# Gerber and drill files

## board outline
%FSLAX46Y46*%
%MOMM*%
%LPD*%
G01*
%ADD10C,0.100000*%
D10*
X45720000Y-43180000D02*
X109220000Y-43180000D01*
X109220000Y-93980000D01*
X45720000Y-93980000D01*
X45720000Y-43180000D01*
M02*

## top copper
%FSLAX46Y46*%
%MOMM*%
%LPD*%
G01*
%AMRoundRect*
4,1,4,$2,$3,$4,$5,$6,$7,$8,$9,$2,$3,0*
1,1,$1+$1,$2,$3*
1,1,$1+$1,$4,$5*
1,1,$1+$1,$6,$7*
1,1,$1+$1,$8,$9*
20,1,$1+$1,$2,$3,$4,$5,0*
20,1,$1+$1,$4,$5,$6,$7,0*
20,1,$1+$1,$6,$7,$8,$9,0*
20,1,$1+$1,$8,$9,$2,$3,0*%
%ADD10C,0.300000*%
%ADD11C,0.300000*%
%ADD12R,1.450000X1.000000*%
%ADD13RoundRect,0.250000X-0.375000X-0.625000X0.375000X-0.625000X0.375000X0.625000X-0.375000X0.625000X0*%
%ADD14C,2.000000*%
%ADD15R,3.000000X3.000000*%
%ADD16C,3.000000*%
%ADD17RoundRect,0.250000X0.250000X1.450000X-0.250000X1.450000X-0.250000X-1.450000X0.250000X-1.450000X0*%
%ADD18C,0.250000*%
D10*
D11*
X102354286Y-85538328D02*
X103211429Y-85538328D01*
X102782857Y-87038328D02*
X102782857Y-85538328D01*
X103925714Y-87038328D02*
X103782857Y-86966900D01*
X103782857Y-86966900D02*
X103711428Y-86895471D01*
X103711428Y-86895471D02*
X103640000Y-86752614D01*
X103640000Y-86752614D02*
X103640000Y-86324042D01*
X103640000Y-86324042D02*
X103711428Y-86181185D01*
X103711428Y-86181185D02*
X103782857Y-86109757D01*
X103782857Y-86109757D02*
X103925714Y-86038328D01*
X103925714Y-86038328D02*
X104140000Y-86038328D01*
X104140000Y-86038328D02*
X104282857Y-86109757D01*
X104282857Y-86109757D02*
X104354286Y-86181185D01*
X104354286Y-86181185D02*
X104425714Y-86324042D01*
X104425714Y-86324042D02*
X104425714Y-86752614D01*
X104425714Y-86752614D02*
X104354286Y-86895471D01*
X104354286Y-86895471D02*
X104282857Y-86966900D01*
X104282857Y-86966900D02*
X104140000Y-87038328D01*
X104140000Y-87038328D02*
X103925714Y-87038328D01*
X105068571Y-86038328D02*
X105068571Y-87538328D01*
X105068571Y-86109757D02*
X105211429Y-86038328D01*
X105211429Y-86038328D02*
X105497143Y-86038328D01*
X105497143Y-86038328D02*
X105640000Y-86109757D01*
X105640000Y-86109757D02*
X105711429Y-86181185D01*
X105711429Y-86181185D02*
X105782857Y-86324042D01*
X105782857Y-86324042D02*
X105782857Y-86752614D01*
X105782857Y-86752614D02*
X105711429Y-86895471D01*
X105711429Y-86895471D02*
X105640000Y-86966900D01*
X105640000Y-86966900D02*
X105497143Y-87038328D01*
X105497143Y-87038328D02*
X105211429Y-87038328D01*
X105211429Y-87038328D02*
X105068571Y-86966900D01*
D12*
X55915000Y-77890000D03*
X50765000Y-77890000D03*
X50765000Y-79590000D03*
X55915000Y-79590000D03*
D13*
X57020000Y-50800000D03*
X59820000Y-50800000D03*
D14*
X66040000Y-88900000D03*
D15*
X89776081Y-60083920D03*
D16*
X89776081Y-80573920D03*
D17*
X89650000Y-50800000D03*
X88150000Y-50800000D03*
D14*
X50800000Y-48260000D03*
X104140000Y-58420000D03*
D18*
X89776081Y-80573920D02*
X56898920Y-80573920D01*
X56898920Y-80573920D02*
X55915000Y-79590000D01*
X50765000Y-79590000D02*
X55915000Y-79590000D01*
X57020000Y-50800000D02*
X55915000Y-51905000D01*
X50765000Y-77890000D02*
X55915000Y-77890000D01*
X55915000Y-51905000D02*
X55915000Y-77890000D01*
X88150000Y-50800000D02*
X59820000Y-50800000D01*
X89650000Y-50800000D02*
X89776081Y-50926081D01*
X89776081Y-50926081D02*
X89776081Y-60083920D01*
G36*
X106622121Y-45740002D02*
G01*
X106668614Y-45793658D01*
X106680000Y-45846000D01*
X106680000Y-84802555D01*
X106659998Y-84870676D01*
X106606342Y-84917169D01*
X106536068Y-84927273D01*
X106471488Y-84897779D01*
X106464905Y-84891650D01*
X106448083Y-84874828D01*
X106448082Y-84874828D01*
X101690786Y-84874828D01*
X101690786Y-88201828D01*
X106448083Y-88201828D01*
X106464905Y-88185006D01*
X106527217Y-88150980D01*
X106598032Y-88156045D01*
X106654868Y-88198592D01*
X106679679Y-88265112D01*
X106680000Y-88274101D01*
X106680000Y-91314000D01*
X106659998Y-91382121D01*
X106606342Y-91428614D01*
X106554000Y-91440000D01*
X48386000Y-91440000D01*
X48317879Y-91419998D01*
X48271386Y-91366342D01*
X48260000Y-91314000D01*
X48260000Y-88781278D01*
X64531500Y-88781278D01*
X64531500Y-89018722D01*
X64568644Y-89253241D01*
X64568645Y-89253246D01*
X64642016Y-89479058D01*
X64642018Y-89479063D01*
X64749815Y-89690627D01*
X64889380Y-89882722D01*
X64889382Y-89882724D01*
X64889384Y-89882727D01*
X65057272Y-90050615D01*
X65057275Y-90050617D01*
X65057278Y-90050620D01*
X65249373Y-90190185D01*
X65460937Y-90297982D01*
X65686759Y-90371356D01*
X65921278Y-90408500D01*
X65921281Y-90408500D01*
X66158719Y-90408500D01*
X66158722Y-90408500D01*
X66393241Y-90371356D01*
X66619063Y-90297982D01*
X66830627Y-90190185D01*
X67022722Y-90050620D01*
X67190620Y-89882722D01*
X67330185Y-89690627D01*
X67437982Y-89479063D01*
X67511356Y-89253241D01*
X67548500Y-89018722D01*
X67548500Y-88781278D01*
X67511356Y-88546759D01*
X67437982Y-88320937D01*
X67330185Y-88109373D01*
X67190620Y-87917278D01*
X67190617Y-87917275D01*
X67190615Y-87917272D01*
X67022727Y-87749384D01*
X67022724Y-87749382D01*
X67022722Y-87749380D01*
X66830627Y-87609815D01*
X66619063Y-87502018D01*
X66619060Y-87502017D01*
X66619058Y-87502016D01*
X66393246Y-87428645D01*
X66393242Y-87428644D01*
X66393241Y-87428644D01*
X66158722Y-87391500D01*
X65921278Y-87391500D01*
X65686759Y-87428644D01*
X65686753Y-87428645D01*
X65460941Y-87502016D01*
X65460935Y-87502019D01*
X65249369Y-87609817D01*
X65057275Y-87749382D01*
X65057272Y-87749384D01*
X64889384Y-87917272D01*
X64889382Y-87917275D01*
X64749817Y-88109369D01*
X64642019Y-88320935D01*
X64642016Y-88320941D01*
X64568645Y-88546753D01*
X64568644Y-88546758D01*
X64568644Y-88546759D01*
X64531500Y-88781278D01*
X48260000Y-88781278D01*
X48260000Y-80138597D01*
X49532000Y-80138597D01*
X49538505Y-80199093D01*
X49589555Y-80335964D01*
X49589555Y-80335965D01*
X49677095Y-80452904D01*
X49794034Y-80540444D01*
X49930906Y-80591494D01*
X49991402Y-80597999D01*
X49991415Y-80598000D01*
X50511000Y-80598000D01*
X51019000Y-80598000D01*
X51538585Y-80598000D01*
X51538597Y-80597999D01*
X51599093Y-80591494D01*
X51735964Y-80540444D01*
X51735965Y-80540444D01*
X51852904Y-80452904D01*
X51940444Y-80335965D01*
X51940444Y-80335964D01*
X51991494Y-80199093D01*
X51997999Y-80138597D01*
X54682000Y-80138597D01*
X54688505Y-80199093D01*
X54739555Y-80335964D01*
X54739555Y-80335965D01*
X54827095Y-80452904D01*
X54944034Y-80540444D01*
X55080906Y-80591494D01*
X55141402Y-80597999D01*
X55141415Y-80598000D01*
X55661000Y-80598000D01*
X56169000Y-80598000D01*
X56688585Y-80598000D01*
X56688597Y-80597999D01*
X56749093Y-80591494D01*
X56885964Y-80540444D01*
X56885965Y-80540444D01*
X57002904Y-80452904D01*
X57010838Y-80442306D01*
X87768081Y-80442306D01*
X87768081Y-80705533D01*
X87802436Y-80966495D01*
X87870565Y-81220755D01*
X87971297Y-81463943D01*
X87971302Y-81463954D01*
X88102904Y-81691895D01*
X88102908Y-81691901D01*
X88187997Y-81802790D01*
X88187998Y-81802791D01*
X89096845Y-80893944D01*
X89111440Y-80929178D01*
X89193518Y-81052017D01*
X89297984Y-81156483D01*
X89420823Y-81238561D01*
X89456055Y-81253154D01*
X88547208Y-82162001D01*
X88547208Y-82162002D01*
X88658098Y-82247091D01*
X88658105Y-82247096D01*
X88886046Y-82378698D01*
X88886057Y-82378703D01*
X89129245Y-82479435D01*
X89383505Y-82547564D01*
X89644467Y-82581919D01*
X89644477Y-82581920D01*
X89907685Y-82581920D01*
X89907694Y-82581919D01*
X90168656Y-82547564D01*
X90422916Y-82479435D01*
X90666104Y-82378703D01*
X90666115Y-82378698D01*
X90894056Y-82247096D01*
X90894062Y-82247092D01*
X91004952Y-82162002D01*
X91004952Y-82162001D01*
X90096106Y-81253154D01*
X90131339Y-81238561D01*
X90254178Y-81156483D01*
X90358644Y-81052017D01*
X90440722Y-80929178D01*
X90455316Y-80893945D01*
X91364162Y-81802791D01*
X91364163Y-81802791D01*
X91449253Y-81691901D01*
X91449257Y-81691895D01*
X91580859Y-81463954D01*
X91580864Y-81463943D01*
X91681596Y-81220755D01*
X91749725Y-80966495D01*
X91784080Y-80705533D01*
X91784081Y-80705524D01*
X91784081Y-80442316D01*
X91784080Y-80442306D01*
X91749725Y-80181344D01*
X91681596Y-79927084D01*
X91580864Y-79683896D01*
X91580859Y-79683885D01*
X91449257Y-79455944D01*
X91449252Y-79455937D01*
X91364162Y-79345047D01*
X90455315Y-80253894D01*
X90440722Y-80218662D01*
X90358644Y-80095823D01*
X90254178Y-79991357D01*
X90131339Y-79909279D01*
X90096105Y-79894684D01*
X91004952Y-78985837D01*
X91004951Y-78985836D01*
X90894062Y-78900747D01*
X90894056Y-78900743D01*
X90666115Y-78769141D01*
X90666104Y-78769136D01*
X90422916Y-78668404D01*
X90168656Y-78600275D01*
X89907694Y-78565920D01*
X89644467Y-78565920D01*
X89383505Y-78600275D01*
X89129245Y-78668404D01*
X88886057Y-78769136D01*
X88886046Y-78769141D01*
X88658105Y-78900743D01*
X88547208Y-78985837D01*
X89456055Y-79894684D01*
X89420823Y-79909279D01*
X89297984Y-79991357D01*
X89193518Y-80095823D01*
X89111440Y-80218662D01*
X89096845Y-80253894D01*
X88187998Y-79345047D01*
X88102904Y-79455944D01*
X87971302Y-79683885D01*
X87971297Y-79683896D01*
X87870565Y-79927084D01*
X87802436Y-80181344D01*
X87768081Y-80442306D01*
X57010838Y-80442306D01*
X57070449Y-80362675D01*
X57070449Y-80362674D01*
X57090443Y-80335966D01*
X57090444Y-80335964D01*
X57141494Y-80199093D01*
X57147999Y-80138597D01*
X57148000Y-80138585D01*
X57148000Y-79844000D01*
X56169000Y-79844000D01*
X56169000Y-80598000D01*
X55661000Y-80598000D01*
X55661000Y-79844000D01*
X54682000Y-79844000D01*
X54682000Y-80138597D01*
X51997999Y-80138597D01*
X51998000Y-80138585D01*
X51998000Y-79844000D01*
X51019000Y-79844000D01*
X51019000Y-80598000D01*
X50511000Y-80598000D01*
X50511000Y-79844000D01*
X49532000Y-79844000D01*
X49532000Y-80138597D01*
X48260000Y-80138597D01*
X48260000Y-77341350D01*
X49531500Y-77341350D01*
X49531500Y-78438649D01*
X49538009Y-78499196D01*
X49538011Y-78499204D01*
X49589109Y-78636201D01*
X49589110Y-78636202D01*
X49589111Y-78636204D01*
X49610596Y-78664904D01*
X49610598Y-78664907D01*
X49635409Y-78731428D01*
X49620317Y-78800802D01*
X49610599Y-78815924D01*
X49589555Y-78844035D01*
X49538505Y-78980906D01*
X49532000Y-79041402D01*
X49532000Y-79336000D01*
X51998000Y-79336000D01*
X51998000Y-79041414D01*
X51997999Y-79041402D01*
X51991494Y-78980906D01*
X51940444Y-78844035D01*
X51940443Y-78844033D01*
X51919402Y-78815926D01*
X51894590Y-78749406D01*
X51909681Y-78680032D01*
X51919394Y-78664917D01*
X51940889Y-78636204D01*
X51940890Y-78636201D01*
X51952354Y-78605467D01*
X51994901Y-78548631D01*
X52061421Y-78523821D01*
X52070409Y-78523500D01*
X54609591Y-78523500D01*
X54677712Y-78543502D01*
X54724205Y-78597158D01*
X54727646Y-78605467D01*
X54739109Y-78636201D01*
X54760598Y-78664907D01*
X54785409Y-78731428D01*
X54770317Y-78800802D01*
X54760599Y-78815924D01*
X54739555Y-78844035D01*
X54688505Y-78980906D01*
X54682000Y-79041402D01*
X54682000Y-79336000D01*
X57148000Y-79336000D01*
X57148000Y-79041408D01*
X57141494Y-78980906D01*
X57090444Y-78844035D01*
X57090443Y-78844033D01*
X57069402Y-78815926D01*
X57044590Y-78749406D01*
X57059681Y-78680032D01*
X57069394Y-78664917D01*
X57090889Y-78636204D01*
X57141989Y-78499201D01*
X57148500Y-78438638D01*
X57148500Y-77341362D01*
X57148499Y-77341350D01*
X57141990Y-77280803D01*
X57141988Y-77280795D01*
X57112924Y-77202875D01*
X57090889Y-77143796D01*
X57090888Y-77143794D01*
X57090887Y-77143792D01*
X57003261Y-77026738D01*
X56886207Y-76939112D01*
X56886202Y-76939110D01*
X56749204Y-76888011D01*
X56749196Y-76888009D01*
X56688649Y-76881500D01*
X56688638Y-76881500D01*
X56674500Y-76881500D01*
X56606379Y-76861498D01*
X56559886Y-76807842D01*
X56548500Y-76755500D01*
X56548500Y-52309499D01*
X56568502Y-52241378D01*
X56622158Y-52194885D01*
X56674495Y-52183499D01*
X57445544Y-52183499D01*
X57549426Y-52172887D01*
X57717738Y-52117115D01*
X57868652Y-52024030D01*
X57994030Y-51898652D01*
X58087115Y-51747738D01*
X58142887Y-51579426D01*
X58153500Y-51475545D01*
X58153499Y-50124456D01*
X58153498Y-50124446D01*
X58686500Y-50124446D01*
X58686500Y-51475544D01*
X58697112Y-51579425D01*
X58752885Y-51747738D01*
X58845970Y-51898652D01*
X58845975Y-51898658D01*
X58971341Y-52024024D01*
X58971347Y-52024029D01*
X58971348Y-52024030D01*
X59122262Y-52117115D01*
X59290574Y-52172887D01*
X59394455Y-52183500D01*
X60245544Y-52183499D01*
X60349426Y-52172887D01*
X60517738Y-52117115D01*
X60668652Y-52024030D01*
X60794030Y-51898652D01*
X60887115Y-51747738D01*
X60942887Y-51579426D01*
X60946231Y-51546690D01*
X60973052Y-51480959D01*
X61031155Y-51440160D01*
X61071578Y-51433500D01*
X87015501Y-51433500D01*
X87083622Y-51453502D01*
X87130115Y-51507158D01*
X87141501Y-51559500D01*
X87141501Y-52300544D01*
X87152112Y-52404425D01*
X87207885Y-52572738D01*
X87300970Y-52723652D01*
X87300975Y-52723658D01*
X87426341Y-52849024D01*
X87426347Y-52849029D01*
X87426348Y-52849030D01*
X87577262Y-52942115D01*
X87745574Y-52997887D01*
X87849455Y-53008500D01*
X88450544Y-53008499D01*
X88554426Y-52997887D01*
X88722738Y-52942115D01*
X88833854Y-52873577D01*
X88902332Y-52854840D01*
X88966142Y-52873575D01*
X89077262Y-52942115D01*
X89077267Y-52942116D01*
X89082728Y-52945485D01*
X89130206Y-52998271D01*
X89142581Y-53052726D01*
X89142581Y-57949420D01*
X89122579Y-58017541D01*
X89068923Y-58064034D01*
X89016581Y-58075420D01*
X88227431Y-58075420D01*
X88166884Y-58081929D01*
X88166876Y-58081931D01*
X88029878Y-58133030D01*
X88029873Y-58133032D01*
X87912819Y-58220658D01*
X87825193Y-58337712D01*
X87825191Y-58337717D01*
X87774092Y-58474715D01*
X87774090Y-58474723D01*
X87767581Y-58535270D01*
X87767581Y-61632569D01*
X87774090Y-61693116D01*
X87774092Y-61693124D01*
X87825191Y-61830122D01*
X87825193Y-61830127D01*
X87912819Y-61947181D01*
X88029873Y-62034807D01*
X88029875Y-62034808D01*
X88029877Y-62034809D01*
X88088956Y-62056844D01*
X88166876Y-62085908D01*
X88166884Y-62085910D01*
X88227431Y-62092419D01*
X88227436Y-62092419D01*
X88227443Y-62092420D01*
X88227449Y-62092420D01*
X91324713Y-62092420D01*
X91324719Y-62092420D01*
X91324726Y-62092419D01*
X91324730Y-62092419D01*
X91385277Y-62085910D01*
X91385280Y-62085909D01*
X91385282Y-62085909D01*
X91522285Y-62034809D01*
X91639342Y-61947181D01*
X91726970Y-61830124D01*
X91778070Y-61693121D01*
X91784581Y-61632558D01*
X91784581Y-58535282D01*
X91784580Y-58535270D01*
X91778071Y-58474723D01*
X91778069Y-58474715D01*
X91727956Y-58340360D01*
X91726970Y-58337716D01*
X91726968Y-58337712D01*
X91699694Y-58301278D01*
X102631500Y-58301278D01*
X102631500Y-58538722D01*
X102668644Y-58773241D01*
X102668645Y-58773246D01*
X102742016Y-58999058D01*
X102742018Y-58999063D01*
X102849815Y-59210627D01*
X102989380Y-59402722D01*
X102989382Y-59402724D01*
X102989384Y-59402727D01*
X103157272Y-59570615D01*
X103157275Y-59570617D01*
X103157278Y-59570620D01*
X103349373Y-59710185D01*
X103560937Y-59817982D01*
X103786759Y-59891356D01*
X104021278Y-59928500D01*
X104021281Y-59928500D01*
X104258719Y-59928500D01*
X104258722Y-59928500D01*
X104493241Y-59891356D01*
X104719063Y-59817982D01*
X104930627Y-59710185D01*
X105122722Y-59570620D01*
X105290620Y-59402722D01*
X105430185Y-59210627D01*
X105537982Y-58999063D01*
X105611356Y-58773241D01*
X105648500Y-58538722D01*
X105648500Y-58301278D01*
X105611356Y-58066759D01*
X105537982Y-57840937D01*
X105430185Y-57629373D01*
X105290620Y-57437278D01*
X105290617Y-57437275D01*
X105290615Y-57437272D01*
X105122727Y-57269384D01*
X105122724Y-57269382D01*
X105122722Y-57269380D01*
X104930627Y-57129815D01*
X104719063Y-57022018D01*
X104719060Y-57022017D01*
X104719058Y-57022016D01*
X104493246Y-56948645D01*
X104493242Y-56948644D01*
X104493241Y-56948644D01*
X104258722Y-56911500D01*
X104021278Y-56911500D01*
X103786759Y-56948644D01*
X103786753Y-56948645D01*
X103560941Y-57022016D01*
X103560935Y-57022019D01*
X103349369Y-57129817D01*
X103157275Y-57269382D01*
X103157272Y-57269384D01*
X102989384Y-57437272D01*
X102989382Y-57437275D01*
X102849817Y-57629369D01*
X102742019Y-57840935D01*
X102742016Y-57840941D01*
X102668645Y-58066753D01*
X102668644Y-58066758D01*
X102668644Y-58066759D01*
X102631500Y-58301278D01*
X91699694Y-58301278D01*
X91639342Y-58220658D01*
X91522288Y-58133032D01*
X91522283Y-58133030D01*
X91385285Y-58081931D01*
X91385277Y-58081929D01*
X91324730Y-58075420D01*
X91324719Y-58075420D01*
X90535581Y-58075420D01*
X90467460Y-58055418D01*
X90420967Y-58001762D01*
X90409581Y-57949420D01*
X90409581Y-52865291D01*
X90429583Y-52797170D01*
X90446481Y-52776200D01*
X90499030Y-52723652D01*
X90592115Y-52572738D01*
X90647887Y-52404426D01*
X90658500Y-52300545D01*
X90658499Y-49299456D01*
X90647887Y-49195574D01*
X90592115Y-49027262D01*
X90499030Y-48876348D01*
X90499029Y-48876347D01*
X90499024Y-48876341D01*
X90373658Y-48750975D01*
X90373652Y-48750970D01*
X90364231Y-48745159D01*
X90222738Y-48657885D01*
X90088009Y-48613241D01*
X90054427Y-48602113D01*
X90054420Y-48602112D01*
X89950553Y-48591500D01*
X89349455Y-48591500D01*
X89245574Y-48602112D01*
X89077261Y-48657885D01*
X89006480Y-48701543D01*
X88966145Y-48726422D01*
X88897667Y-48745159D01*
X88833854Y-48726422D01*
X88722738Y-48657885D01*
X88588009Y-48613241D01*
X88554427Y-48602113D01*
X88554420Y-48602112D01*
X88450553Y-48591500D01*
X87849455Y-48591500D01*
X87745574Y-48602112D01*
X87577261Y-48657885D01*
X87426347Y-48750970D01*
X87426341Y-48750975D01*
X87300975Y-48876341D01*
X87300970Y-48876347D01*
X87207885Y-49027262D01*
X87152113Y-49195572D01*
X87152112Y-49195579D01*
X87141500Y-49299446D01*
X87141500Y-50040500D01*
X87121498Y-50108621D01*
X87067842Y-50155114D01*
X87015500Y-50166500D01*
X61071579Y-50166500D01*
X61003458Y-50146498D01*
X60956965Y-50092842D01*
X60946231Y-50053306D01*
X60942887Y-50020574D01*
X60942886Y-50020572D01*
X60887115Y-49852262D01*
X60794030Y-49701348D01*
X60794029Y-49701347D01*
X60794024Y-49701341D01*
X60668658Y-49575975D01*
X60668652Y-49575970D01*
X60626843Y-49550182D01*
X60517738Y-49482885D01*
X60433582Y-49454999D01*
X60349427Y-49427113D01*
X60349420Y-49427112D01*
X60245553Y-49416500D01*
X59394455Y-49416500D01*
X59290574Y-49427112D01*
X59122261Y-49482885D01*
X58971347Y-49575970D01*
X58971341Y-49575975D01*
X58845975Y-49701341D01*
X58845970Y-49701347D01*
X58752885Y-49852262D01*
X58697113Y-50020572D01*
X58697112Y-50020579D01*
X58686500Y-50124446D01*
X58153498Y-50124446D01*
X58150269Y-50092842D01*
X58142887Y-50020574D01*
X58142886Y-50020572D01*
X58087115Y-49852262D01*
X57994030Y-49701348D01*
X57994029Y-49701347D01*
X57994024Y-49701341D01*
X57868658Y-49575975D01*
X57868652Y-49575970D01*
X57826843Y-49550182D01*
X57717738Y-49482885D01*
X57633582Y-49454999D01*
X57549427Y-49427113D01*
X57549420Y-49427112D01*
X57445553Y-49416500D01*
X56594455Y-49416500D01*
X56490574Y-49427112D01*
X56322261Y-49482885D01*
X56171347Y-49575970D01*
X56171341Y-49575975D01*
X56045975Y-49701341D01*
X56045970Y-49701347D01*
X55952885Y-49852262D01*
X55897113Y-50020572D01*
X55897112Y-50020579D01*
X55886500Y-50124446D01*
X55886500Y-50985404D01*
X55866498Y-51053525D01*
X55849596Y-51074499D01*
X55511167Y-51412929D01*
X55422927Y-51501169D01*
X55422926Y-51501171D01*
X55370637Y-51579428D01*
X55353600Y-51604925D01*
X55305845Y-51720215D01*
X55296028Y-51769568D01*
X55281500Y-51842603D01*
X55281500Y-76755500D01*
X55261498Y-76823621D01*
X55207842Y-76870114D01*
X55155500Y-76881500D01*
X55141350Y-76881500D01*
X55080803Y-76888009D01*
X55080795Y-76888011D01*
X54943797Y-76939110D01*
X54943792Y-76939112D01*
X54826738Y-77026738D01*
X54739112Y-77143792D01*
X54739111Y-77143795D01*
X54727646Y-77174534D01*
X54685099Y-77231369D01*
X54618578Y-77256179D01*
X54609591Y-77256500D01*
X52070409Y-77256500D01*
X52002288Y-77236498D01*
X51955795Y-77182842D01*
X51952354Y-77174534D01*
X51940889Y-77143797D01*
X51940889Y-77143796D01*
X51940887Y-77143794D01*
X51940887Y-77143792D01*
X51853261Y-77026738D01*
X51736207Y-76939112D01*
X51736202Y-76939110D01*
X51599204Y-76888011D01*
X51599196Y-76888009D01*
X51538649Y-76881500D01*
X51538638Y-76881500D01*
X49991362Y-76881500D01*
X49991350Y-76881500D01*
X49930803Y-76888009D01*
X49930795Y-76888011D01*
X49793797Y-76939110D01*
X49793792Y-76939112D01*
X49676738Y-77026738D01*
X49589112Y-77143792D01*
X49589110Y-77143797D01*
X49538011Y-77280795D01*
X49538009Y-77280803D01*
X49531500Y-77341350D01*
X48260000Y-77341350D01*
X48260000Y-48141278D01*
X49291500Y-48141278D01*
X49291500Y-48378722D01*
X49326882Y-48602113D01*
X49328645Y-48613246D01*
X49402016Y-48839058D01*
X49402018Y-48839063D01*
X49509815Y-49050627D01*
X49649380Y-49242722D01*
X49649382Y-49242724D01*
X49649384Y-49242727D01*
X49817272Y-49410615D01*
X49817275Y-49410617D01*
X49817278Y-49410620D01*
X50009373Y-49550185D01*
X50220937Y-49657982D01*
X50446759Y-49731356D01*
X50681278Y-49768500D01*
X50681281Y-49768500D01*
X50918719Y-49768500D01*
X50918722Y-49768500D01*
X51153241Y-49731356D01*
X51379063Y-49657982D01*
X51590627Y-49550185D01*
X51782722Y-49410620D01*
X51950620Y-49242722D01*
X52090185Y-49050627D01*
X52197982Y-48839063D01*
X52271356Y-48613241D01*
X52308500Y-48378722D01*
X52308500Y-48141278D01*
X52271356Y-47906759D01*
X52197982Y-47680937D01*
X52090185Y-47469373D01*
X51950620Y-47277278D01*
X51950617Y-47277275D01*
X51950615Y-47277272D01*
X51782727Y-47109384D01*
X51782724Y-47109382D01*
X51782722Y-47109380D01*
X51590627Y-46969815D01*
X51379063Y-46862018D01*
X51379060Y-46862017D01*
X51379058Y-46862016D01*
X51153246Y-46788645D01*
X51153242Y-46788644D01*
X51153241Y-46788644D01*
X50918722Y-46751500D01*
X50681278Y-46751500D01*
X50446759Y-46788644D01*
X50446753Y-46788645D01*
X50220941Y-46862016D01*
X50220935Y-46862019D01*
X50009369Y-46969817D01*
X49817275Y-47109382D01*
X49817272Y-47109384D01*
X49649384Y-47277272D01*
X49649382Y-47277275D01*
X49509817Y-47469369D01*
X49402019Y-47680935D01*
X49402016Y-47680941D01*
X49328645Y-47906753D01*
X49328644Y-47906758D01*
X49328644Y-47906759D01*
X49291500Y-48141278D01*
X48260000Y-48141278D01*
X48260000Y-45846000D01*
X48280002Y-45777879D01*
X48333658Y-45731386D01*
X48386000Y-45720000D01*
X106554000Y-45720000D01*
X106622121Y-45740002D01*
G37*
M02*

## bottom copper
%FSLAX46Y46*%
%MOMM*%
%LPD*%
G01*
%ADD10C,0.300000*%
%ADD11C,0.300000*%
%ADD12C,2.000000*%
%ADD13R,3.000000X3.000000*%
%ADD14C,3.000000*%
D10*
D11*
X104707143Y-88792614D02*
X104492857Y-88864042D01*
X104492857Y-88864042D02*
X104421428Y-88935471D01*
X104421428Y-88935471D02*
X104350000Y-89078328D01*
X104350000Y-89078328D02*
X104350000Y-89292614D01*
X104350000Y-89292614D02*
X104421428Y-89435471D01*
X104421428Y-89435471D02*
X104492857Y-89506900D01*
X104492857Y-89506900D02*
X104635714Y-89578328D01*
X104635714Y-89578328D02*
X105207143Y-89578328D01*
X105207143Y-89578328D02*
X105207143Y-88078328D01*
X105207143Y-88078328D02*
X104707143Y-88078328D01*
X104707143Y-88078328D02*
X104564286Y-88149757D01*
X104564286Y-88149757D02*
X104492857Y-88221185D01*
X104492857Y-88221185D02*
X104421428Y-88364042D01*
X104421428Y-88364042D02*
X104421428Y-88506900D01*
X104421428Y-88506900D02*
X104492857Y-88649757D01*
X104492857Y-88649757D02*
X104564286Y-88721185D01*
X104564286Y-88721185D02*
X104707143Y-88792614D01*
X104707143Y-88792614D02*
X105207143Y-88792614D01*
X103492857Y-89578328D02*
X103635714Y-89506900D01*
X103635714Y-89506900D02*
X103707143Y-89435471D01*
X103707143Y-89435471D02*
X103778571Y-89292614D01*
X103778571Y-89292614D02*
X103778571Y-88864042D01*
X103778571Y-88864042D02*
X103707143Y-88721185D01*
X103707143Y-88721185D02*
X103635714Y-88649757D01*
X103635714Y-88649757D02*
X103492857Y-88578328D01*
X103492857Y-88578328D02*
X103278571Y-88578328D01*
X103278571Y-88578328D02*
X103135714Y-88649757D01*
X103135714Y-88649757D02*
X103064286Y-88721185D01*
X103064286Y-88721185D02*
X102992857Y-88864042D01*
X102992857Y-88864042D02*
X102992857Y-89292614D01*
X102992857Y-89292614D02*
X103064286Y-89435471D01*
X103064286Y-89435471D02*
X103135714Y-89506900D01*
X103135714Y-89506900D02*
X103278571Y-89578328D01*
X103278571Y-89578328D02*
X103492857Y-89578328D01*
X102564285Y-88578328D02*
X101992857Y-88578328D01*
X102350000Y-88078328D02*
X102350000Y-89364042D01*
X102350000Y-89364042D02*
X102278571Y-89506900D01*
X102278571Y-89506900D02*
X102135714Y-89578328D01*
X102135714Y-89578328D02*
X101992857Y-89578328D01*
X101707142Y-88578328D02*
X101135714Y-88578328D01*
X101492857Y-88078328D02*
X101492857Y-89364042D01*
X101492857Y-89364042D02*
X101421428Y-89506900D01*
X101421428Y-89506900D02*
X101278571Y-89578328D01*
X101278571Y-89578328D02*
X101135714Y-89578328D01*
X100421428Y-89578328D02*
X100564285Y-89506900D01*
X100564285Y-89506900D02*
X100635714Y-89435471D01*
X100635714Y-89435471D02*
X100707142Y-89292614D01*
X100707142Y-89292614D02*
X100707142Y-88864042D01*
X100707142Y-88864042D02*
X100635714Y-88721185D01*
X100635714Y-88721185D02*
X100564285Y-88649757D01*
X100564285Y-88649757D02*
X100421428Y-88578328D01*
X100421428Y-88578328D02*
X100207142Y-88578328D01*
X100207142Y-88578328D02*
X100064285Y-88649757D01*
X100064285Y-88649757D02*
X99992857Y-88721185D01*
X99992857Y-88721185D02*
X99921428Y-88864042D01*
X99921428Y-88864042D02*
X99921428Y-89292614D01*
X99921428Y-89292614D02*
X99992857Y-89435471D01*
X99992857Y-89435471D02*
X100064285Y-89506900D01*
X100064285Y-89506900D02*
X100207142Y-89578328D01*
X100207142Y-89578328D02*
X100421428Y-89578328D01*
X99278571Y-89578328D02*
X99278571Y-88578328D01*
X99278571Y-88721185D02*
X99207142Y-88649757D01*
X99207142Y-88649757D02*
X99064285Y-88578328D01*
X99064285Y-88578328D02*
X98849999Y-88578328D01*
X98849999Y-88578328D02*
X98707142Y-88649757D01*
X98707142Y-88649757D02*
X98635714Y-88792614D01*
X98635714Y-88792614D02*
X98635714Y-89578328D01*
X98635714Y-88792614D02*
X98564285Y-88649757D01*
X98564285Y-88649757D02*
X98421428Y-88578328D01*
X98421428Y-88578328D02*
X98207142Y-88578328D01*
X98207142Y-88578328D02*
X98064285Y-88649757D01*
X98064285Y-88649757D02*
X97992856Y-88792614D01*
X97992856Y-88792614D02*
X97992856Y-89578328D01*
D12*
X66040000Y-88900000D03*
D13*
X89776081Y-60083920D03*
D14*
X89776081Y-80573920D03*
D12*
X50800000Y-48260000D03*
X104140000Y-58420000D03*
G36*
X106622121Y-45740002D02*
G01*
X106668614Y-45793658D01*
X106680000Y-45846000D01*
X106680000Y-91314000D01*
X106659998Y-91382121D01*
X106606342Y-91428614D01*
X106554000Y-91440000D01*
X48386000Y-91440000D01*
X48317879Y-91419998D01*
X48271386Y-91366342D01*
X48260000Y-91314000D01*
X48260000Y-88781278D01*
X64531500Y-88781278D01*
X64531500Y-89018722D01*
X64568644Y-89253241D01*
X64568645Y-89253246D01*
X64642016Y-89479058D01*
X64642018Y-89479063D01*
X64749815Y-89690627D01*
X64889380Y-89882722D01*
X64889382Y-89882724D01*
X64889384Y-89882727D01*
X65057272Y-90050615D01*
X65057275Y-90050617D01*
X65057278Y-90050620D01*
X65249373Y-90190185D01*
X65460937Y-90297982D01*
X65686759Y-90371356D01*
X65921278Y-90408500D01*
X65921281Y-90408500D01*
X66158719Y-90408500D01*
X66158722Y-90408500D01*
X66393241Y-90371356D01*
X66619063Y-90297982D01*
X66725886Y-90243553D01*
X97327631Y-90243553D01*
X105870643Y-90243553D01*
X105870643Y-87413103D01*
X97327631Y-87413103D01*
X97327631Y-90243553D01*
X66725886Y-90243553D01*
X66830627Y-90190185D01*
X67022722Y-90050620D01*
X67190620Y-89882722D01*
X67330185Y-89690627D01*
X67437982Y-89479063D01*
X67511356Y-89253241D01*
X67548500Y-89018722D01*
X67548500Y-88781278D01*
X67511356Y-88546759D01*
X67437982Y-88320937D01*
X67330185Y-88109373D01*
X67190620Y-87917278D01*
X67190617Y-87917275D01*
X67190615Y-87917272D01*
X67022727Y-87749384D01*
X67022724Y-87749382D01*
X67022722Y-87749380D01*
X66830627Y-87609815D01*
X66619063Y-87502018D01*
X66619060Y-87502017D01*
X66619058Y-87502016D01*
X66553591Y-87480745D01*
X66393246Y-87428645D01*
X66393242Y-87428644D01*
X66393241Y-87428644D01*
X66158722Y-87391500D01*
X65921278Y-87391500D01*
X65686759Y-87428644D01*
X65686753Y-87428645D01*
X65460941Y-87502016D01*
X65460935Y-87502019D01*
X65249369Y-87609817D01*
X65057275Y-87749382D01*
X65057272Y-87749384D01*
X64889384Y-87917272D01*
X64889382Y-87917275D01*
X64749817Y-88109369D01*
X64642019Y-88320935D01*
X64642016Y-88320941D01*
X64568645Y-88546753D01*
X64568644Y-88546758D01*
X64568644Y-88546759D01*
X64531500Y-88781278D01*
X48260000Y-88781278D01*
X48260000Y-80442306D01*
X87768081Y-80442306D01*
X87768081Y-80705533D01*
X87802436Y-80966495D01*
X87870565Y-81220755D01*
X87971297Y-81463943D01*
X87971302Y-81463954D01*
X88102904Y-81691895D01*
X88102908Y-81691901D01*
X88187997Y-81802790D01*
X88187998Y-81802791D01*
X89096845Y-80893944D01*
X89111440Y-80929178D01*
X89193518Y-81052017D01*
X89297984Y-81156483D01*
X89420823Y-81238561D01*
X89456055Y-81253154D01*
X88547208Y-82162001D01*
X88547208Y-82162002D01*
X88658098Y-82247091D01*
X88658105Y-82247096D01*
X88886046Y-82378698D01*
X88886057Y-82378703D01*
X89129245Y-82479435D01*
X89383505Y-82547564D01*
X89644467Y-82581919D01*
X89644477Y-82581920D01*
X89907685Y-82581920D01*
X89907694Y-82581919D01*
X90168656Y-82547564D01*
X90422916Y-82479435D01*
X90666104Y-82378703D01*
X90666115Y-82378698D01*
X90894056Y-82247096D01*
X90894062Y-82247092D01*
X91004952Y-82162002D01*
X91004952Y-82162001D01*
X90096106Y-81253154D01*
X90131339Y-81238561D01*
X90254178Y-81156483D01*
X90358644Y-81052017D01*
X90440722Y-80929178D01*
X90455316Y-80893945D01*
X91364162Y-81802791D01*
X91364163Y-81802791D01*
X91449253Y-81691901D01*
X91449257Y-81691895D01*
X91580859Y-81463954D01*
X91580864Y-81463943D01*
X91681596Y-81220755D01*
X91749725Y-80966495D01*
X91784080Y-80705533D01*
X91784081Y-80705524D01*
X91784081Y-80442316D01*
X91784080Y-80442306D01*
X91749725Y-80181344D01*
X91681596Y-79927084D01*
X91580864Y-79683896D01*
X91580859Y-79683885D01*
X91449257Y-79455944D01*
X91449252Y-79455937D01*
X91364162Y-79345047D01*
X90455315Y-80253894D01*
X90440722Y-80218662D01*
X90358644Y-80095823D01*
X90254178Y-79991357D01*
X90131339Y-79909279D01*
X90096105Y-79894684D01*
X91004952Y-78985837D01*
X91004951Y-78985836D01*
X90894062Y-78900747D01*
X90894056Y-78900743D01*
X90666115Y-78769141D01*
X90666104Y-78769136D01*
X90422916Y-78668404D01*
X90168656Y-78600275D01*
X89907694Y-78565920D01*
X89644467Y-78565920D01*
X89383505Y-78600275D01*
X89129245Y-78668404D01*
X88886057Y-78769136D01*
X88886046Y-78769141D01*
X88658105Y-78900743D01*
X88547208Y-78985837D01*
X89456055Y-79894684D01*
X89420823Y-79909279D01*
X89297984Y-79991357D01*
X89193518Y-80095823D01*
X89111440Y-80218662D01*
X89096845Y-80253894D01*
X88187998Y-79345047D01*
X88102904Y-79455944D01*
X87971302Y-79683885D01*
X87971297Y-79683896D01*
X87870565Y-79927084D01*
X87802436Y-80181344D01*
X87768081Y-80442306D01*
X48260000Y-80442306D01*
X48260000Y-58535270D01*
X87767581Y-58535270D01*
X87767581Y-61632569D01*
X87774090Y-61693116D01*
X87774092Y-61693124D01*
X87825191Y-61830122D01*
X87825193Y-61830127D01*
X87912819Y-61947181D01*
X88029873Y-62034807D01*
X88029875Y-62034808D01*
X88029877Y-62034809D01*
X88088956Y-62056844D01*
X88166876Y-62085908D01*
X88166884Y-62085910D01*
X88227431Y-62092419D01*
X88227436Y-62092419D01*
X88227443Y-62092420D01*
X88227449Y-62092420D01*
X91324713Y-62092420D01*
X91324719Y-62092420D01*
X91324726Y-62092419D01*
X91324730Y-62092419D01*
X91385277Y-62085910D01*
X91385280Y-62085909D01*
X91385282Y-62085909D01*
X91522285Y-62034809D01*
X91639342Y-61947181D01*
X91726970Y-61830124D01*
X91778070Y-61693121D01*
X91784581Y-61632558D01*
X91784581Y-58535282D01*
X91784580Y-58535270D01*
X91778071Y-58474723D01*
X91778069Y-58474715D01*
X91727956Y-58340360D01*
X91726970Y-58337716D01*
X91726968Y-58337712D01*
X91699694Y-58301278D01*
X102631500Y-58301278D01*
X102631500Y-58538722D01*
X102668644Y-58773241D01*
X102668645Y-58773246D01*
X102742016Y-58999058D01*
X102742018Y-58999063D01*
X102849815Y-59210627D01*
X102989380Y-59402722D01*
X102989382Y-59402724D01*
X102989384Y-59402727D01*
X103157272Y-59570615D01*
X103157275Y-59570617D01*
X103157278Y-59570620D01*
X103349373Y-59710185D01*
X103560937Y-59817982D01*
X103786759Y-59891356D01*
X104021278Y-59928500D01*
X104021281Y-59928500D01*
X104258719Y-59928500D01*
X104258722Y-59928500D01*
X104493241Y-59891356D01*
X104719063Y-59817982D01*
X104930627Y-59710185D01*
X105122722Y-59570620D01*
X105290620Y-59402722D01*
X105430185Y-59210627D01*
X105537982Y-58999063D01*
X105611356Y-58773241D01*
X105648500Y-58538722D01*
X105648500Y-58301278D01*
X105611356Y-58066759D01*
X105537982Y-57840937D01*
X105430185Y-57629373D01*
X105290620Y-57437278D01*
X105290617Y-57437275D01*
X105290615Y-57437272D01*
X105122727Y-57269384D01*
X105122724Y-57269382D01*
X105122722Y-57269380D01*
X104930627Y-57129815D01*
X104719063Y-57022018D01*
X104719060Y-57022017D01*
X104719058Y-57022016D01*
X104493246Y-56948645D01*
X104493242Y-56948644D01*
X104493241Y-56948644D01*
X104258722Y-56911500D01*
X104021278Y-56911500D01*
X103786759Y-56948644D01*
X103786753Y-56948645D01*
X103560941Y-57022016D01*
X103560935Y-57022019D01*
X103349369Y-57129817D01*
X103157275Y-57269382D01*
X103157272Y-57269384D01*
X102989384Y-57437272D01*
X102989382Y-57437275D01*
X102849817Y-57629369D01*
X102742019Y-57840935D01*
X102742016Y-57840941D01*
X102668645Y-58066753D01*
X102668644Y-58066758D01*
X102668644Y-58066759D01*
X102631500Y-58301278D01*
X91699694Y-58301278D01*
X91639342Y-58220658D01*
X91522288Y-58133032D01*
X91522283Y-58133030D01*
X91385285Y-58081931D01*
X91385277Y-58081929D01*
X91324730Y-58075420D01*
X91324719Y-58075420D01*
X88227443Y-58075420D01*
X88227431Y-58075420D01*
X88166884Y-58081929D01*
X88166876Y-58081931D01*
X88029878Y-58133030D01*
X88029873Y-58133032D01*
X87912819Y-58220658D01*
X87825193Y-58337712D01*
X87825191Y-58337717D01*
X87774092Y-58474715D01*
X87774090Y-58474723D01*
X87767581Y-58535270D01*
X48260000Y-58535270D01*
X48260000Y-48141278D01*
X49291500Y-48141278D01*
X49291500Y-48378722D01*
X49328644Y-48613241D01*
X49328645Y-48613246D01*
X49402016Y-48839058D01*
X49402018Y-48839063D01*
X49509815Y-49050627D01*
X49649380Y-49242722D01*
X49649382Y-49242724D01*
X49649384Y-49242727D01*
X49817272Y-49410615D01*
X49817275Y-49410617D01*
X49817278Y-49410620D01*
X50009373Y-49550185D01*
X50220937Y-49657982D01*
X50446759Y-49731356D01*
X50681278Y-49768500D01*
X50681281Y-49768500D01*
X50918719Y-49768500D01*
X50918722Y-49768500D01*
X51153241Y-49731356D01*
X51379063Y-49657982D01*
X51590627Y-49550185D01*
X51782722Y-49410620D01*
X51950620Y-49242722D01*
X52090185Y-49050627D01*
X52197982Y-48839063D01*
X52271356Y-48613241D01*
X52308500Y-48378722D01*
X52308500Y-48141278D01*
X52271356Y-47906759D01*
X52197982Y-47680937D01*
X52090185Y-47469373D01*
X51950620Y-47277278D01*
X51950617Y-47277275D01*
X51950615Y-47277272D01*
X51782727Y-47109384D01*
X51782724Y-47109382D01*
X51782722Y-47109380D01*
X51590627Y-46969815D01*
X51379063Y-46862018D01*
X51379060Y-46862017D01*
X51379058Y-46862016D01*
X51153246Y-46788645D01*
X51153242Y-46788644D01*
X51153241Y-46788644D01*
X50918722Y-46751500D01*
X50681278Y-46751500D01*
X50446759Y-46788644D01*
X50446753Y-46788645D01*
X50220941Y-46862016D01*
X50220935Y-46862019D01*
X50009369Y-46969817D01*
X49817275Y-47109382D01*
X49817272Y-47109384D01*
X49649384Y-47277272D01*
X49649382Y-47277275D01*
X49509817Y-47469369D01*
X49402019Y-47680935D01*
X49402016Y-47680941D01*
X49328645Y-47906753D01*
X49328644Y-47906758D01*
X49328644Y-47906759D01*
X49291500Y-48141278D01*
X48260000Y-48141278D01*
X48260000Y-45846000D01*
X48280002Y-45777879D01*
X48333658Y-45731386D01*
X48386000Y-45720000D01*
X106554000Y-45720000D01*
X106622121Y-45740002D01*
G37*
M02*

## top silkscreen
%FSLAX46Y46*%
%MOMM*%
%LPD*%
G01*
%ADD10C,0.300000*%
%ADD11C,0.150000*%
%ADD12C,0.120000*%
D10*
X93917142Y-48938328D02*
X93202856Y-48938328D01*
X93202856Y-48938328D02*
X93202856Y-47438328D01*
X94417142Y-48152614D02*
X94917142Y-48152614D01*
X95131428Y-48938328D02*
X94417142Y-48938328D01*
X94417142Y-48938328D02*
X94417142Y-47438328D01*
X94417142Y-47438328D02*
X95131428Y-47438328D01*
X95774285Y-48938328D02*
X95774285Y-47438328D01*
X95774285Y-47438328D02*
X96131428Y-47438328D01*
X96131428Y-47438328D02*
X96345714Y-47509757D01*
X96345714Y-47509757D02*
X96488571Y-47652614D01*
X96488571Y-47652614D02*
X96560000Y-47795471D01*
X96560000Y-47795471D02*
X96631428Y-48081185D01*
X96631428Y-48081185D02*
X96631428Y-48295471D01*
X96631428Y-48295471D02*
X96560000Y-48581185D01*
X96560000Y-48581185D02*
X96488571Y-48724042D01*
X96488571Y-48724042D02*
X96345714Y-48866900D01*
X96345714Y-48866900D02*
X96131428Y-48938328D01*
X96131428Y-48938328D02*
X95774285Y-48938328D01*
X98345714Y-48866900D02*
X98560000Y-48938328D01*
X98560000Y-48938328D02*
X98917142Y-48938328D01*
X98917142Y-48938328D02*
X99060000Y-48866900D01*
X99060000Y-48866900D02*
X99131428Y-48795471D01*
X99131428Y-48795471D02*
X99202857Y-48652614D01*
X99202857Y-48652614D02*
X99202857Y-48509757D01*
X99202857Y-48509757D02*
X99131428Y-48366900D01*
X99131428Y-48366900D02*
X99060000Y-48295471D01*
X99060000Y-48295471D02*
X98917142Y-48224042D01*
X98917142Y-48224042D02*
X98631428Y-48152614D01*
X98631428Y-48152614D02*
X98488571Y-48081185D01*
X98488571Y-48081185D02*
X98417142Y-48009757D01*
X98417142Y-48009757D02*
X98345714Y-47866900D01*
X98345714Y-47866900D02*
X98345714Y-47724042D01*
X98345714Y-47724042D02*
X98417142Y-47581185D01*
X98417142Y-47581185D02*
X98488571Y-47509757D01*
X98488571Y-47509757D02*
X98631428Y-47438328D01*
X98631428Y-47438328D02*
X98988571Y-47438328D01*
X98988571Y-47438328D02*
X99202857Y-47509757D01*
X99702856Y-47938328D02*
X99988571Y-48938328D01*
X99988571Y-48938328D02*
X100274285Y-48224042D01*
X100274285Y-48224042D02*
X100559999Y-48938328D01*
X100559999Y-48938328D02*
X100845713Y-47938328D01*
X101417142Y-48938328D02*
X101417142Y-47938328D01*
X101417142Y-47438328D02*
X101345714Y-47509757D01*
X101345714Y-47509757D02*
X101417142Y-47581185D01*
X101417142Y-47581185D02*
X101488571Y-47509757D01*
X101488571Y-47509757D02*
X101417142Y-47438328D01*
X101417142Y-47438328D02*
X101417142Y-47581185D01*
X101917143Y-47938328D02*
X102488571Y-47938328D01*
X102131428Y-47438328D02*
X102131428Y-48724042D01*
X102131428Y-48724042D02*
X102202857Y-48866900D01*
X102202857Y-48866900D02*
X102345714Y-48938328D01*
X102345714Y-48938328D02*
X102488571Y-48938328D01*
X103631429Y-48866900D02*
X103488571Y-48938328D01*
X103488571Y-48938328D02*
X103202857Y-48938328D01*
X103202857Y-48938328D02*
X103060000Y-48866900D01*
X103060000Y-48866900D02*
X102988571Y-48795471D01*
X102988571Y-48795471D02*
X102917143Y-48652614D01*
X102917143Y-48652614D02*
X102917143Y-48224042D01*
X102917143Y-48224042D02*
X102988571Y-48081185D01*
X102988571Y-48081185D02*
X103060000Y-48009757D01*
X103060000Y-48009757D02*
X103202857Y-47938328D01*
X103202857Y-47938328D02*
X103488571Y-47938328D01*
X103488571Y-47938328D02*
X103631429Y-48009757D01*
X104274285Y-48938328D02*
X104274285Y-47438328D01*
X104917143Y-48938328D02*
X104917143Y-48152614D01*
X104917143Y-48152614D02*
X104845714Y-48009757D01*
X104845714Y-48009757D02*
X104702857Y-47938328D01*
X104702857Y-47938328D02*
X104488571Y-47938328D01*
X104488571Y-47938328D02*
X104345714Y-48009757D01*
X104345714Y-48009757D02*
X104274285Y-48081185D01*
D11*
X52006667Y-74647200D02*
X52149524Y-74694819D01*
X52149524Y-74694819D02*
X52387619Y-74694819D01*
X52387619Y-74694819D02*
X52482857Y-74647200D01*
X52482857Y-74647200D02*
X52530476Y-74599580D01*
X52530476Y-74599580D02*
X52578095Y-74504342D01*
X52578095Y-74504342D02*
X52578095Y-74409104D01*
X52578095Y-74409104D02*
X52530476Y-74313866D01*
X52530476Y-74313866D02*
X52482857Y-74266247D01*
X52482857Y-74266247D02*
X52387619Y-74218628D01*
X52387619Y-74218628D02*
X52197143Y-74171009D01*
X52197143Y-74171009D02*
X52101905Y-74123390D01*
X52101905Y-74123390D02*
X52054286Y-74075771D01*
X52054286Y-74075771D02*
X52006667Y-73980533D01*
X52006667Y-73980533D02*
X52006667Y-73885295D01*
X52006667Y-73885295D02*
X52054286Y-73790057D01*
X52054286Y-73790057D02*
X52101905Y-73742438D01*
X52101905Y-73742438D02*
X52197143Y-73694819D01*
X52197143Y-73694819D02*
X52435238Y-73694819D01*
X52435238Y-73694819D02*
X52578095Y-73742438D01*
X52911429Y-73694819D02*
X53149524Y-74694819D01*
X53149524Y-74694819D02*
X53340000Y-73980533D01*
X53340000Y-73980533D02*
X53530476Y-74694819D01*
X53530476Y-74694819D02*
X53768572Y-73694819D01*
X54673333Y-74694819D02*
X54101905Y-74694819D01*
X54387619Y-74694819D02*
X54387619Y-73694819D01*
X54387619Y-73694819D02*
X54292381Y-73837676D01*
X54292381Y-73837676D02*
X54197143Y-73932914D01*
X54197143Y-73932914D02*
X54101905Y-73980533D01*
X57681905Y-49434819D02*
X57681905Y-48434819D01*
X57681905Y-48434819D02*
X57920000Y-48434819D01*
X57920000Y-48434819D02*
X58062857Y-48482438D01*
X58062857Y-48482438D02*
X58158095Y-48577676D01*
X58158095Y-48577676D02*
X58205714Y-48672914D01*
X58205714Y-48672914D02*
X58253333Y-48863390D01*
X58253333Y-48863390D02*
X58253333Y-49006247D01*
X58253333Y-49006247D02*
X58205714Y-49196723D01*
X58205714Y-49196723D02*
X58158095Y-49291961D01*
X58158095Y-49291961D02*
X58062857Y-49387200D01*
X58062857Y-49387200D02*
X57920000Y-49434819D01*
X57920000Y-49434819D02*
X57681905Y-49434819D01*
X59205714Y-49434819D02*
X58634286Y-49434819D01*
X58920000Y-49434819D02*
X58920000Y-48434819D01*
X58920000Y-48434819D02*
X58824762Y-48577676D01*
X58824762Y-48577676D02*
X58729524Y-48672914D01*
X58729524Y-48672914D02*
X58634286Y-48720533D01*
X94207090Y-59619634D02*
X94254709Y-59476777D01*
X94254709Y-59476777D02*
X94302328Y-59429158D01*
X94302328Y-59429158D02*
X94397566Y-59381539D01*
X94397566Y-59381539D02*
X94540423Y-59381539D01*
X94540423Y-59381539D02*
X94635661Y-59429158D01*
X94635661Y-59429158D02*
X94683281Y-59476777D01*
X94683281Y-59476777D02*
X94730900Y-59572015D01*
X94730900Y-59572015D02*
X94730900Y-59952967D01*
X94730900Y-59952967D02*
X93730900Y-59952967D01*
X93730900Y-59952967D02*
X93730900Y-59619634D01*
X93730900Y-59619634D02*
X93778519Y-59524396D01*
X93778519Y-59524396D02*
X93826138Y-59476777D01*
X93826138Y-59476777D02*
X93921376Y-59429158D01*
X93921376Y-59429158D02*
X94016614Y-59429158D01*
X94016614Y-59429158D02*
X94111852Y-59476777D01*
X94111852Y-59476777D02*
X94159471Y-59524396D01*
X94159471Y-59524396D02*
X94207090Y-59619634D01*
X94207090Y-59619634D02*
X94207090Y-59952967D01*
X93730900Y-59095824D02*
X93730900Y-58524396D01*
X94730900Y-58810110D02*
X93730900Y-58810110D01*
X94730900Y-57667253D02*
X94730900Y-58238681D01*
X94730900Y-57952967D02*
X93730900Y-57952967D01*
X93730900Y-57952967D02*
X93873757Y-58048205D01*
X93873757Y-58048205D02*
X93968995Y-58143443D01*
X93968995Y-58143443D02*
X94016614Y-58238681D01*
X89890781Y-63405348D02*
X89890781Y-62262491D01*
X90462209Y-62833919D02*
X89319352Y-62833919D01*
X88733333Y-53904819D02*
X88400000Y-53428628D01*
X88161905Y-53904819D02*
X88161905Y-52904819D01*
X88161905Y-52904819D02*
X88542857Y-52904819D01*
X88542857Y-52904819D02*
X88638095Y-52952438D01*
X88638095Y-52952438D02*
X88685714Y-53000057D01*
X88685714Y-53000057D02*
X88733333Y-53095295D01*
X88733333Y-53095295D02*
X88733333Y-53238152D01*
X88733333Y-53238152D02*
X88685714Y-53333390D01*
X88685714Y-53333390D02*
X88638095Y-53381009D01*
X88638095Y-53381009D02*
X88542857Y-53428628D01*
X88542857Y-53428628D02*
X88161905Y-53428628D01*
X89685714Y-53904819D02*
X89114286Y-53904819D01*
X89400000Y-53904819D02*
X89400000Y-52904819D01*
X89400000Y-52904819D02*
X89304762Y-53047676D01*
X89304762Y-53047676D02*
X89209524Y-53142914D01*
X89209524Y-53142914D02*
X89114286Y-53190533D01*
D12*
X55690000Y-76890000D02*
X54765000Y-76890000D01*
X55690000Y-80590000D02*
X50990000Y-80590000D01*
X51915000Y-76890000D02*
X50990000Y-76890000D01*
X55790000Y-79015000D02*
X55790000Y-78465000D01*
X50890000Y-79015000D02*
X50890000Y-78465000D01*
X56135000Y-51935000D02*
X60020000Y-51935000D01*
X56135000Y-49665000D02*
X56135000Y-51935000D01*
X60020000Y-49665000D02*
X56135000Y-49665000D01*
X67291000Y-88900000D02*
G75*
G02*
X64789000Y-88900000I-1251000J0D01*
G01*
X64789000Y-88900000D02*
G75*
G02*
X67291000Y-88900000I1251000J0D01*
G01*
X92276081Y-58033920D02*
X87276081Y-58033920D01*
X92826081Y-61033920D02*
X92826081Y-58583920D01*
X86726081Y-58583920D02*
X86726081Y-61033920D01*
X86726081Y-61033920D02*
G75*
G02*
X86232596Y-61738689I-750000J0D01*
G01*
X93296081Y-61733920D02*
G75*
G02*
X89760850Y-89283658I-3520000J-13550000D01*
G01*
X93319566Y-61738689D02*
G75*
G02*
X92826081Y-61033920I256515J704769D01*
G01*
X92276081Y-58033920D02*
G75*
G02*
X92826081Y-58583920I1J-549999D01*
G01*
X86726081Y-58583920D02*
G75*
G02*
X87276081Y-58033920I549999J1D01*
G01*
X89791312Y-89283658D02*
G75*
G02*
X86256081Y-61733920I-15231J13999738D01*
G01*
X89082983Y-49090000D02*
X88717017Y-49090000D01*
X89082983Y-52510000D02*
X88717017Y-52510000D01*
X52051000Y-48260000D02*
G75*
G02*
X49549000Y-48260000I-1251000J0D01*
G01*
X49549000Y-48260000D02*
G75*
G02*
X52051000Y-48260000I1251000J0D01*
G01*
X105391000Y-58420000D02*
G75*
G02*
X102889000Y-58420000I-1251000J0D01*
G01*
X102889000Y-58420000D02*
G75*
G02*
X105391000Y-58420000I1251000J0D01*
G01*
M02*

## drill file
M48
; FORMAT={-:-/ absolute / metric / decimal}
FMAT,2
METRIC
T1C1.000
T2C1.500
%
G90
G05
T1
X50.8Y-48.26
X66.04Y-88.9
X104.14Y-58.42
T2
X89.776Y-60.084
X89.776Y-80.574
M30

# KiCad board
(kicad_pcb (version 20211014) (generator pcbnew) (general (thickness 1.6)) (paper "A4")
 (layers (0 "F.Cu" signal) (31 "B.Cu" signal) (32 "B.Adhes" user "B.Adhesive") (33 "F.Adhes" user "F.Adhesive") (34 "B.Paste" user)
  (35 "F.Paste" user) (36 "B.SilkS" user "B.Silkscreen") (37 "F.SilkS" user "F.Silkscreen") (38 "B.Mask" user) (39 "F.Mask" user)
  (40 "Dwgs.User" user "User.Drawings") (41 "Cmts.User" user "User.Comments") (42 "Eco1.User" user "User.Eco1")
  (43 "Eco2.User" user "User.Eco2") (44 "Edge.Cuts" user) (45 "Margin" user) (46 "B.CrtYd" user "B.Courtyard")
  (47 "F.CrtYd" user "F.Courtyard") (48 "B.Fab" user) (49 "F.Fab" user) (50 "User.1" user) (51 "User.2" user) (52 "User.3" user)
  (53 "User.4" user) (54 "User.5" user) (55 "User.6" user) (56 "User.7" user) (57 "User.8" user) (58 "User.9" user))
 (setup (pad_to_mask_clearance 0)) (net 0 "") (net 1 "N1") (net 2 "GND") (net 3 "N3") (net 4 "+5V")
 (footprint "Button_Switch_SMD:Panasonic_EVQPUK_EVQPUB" (layer "F.Cu") (at 53.34 78.74)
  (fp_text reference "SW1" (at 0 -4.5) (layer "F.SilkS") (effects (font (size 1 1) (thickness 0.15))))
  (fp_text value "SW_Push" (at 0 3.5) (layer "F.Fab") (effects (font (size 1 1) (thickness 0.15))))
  (fp_line (start 2.35 -1.85) (end 1.425 -1.85) (layer "F.SilkS") (width 0.12))
  (fp_line (start 2.35 1.85) (end -2.35 1.85) (layer "F.SilkS") (width 0.12))
  (fp_line (start -1.425 -1.85) (end -2.35 -1.85) (layer "F.SilkS") (width 0.12))
  (fp_line (start 2.45 0.275) (end 2.45 -0.275) (layer "F.SilkS") (width 0.12))
  (fp_line (start -2.45 0.275) (end -2.45 -0.275) (layer "F.SilkS") (width 0.12))
  (pad "1" smd rect (at 2.575 -0.85 180) (size 1.45 1) (layers "F.Cu" "F.Paste" "F.Mask") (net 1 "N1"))
  (pad "1" smd rect (at -2.575 -0.85 180) (size 1.45 1) (layers "F.Cu" "F.Paste" "F.Mask") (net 1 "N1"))
  (pad "2" smd rect (at -2.575 0.85 180) (size 1.45 1) (layers "F.Cu" "F.Paste" "F.Mask") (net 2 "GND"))
  (pad "2" smd rect (at 2.575 0.85 180) (size 1.45 1) (layers "F.Cu" "F.Paste" "F.Mask") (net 2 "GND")))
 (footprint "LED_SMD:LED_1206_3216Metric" (layer "F.Cu") (at 58.42 50.8)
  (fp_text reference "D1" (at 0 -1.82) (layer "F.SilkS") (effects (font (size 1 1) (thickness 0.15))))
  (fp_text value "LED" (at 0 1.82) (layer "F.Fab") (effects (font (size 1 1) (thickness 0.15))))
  (fp_line (start -2.285 1.135) (end 1.6 1.135) (layer "F.SilkS") (width 0.12))
  (fp_line (start -2.285 -1.135) (end -2.285 1.135) (layer "F.SilkS") (width 0.12))
  (fp_line (start 1.6 -1.135) (end -2.285 -1.135) (layer "F.SilkS") (width 0.12))
  (pad "1" smd roundrect (at -1.4 0) (size 1.25 1.75) (layers "F.Cu" "F.Paste" "F.Mask") (roundrect_rratio 0.2) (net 1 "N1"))
  (pad "2" smd roundrect (at 1.4 0) (size 1.25 1.75) (layers "F.Cu" "F.Paste" "F.Mask") (roundrect_rratio 0.2) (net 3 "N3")))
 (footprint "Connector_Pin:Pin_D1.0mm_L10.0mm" (layer "F.Cu") (at 66.04 88.9)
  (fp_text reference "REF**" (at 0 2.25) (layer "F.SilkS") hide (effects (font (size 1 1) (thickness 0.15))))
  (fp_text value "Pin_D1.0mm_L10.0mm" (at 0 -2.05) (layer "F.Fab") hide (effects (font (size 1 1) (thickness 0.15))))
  (fp_circle (center 0 0) (end 1.25 0.05) (layer "F.SilkS") (width 0.12) (fill none))
  (pad "1" thru_hole circle (at 0 0) (size 2 2) (drill 1) (layers *.Cu *.Mask)))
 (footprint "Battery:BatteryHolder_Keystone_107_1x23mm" (layer "F.Cu") (at 89.776081 60.08392 -90)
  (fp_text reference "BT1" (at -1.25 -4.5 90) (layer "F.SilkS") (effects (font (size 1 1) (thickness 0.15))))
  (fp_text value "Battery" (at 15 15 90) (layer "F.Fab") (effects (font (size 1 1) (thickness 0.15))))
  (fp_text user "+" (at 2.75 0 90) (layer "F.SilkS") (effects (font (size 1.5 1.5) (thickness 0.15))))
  (fp_line (start -2.05 -2.5) (end -2.05 2.5) (layer "F.SilkS") (width 0.12))
  (fp_line (start 0.95 -3.05) (end -1.5 -3.05) (layer "F.SilkS") (width 0.12))
  (fp_line (start -1.5 3.05) (end 0.95 3.05) (layer "F.SilkS") (width 0.12))
  (fp_arc (start 0.95 3.05) (mid 1.380182 3.185636) (end 1.654769 3.543485) (layer "F.SilkS") (width 0.12))
  (fp_arc (start 1.65 -3.52) (mid 16.981862 -13.885887) (end 29.199738 0.015231) (layer "F.SilkS") (width 0.12))
  (fp_arc (start 1.654769 -3.543485) (mid 1.380182 -3.185636) (end 0.95 -3.05) (layer "F.SilkS") (width 0.12))
  (fp_arc (start -2.05 -2.5) (mid -1.888909 -2.888909) (end -1.5 -3.05) (layer "F.SilkS") (width 0.12))
  (fp_arc (start -1.5 3.05) (mid -1.888909 2.888909) (end -2.05 2.5) (layer "F.SilkS") (width 0.12))
  (fp_arc (start 29.199738 -0.015231) (mid 16.981862 13.885887) (end 1.65 3.52) (layer "F.SilkS") (width 0.12))
  (pad "1" thru_hole rect (at 0 0 270) (size 3 3) (drill 1.5) (layers *.Cu *.Mask) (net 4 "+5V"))
  (pad "2" thru_hole circle (at 20.49 0 270) (size 3 3) (drill 1.5) (layers *.Cu *.Mask) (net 2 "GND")))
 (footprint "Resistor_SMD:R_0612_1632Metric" (layer "F.Cu") (at 88.9 50.8 180)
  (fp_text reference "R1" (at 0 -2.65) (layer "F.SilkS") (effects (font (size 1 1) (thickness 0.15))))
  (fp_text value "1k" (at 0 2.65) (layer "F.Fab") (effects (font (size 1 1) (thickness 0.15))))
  (fp_line (start -0.182983 1.71) (end 0.182983 1.71) (layer "F.SilkS") (width 0.12))
  (fp_line (start -0.182983 -1.71) (end 0.182983 -1.71) (layer "F.SilkS") (width 0.12))
  (pad "1" smd roundrect (at -0.75 0 180) (size 1 3.4) (layers "F.Cu" "F.Paste" "F.Mask") (roundrect_rratio 0.25) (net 4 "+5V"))
  (pad "2" smd roundrect (at 0.75 0 180) (size 1 3.4) (layers "F.Cu" "F.Paste" "F.Mask") (roundrect_rratio 0.25) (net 3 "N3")))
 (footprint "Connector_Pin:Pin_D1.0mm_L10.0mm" (layer "F.Cu") (at 50.8 48.26)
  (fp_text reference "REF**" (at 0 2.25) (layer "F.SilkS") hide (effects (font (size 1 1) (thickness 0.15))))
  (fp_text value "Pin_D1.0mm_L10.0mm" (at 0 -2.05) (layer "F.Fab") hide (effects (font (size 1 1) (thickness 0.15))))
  (fp_circle (center 0 0) (end 1.25 0.05) (layer "F.SilkS") (width 0.12) (fill none))
  (pad "1" thru_hole circle (at 0 0) (size 2 2) (drill 1) (layers *.Cu *.Mask)))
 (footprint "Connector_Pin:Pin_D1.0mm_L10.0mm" (layer "F.Cu") (at 104.14 58.42)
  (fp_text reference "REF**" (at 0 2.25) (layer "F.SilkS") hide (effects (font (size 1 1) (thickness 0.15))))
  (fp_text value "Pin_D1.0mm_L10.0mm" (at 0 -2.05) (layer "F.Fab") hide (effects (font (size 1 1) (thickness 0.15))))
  (fp_circle (center 0 0) (end 1.25 0.05) (layer "F.SilkS") (width 0.12) (fill none))
  (pad "1" thru_hole circle (at 0 0) (size 2 2) (drill 1) (layers *.Cu *.Mask)))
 (gr_rect (start 109.22 93.98) (end 45.72 43.18) (layer "Edge.Cuts") (width 0.1) (fill none))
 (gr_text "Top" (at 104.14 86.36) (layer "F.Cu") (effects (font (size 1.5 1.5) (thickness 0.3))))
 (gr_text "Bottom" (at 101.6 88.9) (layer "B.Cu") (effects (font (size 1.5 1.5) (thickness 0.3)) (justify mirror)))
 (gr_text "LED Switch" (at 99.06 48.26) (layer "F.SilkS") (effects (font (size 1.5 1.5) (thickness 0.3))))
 (segment (start 89.776081 80.57392) (end 56.89892 80.57392) (width 0.25) (layer "F.Cu") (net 2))
 (segment (start 56.89892 80.57392) (end 55.915 79.59) (width 0.25) (layer "F.Cu") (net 2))
 (segment (start 50.765 79.59) (end 55.915 79.59) (width 0.25) (layer "F.Cu") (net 2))
 (segment (start 57.02 50.8) (end 55.915 51.905) (width 0.25) (layer "F.Cu") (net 1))
 (segment (start 50.765 77.89) (end 55.915 77.89) (width 0.25) (layer "F.Cu") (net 1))
 (segment (start 55.915 51.905) (end 55.915 77.89) (width 0.25) (layer "F.Cu") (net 1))
 (segment (start 88.15 50.8) (end 59.82 50.8) (width 0.25) (layer "F.Cu") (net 3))
 (segment (start 89.65 50.8) (end 89.776081 50.926081) (width 0.25) (layer "F.Cu") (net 4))
 (segment (start 89.776081 50.926081) (end 89.776081 60.08392) (width 0.25) (layer "F.Cu") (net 4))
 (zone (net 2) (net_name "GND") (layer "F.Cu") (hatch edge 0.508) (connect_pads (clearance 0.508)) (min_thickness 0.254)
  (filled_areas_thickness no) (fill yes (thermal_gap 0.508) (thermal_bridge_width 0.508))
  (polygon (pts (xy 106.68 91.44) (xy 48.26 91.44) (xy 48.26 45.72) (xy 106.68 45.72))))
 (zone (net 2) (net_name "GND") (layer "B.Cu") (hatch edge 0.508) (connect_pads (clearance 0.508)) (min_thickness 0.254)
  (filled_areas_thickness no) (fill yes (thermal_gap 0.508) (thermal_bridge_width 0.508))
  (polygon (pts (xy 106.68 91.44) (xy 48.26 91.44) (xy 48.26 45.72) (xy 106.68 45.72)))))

